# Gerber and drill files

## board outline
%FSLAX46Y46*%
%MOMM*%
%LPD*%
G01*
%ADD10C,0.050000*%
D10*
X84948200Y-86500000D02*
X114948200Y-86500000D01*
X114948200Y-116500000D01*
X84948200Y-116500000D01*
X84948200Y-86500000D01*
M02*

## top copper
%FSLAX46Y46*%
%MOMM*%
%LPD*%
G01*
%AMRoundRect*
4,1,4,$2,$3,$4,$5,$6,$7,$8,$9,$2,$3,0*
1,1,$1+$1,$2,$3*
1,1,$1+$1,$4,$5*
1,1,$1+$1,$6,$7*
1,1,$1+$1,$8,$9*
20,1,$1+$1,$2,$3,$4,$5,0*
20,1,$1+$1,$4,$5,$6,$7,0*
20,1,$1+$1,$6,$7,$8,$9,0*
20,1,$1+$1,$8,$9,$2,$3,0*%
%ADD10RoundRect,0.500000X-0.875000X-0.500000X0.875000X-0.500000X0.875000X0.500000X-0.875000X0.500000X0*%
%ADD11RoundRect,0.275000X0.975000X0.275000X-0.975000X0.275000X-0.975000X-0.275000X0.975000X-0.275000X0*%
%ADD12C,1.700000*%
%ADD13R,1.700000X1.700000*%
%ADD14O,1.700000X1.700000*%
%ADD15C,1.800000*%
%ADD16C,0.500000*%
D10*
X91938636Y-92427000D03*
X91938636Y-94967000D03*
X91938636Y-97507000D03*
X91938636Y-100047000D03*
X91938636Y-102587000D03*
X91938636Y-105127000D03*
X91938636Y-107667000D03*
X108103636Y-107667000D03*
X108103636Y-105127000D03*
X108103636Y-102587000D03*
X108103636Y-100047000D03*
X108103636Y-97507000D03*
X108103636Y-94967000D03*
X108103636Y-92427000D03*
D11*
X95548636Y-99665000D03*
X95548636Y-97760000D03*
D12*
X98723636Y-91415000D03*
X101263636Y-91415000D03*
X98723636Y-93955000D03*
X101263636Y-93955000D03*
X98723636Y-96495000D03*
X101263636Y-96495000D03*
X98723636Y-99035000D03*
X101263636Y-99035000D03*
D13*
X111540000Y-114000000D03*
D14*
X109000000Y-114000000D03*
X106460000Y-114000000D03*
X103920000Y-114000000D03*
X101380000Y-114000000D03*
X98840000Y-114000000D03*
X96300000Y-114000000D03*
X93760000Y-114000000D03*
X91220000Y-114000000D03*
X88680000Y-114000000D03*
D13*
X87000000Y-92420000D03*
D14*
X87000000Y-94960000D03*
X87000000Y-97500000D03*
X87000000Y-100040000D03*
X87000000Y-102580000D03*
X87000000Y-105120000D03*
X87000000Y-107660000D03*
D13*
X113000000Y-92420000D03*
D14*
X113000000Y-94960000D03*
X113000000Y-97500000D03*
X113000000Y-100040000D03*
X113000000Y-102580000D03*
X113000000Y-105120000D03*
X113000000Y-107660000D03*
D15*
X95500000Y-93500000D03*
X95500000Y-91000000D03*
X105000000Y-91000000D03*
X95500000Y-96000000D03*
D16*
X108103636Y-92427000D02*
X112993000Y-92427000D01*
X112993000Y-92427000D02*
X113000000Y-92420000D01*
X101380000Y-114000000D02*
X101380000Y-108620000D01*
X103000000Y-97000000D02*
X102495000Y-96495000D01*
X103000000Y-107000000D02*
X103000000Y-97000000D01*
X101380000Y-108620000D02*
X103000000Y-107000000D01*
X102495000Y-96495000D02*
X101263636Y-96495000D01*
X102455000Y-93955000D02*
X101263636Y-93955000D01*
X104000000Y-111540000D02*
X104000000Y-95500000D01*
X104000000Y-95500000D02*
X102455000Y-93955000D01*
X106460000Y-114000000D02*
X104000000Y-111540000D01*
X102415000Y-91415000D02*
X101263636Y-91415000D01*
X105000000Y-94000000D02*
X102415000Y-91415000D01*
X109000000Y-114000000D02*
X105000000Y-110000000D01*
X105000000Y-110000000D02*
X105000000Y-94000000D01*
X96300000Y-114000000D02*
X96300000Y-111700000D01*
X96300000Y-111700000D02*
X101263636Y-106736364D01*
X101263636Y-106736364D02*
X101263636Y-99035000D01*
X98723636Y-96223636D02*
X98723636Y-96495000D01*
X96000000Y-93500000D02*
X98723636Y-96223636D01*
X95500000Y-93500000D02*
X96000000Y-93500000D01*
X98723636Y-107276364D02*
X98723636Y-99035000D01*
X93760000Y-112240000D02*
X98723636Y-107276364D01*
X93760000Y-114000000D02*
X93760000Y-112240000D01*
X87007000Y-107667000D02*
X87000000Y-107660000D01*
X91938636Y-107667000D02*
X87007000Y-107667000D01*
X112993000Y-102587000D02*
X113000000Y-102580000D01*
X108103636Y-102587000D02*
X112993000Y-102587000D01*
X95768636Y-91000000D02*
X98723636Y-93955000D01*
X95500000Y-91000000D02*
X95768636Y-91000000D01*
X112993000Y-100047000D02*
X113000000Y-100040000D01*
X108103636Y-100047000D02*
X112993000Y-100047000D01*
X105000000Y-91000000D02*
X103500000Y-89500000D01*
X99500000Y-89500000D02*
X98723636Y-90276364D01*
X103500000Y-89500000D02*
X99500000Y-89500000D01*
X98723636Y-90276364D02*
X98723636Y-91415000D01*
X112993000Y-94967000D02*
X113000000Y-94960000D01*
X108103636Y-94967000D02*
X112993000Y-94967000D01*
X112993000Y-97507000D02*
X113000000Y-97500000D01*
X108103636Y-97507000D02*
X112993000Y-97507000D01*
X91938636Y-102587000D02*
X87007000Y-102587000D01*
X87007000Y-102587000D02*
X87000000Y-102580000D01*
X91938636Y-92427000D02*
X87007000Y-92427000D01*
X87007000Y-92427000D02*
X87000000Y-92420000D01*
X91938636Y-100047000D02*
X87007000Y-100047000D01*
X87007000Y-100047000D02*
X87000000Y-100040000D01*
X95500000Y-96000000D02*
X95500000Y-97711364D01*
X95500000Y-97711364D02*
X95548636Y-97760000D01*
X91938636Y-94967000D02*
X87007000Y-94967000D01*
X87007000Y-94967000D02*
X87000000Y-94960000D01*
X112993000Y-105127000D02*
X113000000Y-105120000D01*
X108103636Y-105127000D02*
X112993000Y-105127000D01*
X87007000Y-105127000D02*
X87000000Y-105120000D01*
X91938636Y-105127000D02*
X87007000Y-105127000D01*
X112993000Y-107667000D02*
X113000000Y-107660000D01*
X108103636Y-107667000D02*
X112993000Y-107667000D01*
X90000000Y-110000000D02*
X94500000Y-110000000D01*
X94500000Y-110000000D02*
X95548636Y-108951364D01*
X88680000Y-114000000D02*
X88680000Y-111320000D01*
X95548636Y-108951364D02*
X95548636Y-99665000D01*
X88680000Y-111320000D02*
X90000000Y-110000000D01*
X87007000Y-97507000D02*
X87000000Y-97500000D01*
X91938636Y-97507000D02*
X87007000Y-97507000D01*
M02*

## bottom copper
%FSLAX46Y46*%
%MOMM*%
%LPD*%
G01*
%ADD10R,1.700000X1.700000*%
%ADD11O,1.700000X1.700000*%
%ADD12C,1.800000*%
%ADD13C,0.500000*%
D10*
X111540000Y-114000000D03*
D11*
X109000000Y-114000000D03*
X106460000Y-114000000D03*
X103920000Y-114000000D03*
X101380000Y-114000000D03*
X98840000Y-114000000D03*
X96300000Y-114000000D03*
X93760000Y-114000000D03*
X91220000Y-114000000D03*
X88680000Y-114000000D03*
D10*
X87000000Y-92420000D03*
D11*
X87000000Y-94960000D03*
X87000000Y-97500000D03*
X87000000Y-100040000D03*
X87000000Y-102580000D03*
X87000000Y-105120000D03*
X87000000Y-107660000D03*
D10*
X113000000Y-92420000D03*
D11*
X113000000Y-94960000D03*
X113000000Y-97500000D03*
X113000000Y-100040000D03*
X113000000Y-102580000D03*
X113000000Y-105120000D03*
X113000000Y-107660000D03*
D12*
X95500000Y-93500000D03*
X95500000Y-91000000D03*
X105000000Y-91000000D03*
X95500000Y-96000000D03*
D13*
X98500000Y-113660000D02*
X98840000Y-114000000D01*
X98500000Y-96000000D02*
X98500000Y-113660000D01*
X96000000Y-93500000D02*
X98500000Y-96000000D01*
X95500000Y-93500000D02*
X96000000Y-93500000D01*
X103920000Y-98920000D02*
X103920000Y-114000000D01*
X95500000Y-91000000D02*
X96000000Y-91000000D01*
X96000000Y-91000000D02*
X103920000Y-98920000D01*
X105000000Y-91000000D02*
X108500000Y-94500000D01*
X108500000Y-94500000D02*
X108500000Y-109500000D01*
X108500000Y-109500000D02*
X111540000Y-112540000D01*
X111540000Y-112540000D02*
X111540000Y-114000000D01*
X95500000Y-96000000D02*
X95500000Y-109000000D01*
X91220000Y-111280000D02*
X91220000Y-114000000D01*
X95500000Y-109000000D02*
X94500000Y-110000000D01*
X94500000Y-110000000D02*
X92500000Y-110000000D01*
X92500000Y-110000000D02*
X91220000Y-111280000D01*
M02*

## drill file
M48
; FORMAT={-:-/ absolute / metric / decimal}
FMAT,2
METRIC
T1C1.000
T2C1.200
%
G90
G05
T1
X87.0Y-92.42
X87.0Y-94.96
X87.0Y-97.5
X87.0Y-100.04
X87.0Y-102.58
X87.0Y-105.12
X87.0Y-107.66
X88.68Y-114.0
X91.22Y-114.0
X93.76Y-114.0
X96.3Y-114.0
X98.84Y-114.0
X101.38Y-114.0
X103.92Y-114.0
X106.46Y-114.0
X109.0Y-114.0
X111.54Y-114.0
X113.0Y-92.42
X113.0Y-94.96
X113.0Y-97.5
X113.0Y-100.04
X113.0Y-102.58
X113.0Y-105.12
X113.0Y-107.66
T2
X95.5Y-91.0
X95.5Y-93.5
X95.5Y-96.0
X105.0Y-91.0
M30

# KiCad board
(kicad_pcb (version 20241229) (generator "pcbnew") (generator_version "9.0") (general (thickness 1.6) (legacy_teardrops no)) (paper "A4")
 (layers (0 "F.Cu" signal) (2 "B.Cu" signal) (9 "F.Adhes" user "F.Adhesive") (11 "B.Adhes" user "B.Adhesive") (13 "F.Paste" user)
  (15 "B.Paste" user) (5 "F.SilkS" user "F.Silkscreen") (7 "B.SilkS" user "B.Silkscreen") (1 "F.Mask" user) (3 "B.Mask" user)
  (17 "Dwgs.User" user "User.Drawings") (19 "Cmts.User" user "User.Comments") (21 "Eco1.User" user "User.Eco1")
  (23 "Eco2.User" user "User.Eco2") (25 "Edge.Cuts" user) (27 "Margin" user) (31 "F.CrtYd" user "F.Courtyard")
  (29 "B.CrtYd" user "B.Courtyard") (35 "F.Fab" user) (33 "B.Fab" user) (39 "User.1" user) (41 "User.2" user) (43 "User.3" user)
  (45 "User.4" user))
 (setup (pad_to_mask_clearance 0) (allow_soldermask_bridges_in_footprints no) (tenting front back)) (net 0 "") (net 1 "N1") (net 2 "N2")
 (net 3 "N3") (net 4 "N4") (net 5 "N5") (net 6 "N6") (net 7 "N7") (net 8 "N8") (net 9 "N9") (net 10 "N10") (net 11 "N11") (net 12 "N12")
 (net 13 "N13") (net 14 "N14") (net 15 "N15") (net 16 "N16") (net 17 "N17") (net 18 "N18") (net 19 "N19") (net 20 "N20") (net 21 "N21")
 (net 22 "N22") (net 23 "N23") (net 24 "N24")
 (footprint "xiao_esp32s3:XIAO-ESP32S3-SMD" (layer "F.Cu") (at 100 100)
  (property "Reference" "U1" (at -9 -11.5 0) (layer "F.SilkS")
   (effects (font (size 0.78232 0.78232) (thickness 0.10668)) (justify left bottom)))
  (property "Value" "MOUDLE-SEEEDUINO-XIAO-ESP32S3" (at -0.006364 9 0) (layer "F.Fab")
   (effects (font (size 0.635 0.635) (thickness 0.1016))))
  (pad "1" smd roundrect (at -8.061364 -7.573) (size 2.75 2) (layers "F.Cu" "F.Mask" "F.Paste") (roundrect_rratio 0.25) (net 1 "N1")
   (solder_mask_margin 0.0508) (thermal_bridge_angle 45))
  (pad "2" smd roundrect (at -8.061364 -5.033) (size 2.75 2) (layers "F.Cu" "F.Mask" "F.Paste") (roundrect_rratio 0.25) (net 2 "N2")
   (solder_mask_margin 0.0508) (thermal_bridge_angle 45))
  (pad "3" smd roundrect (at -8.061364 -2.493) (size 2.75 2) (layers "F.Cu" "F.Mask" "F.Paste") (roundrect_rratio 0.25) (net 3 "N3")
   (solder_mask_margin 0.0508) (thermal_bridge_angle 45))
  (pad "4" smd roundrect (at -8.061364 0.047) (size 2.75 2) (layers "F.Cu" "F.Mask" "F.Paste") (roundrect_rratio 0.25) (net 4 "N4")
   (solder_mask_margin 0.0508) (thermal_bridge_angle 45))
  (pad "5" smd roundrect (at -8.061364 2.587) (size 2.75 2) (layers "F.Cu" "F.Mask" "F.Paste") (roundrect_rratio 0.25) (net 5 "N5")
   (solder_mask_margin 0.0508) (thermal_bridge_angle 45))
  (pad "6" smd roundrect (at -8.061364 5.127) (size 2.75 2) (layers "F.Cu" "F.Mask" "F.Paste") (roundrect_rratio 0.25) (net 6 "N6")
   (solder_mask_margin 0.0508) (thermal_bridge_angle 45))
  (pad "7" smd roundrect (at -8.061364 7.667) (size 2.75 2) (layers "F.Cu" "F.Mask" "F.Paste") (roundrect_rratio 0.25) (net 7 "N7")
   (solder_mask_margin 0.0508) (thermal_bridge_angle 45))
  (pad "8" smd roundrect (at 8.103636 7.667) (size 2.75 2) (layers "F.Cu" "F.Mask" "F.Paste") (roundrect_rratio 0.25) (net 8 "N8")
   (solder_mask_margin 0.0508) (thermal_bridge_angle 45))
  (pad "9" smd roundrect (at 8.103636 5.127) (size 2.75 2) (layers "F.Cu" "F.Mask" "F.Paste") (roundrect_rratio 0.25) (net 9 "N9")
   (solder_mask_margin 0.0508) (thermal_bridge_angle 45))
  (pad "10" smd roundrect (at 8.103636 2.587) (size 2.75 2) (layers "F.Cu" "F.Mask" "F.Paste") (roundrect_rratio 0.25) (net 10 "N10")
   (solder_mask_margin 0.0508) (thermal_bridge_angle 45))
  (pad "11" smd roundrect (at 8.103636 0.047) (size 2.75 2) (layers "F.Cu" "F.Mask" "F.Paste") (roundrect_rratio 0.25) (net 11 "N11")
   (solder_mask_margin 0.0508) (thermal_bridge_angle 45))
  (pad "12" smd roundrect (at 8.103636 -2.493) (size 2.75 2) (layers "F.Cu" "F.Mask" "F.Paste") (roundrect_rratio 0.25) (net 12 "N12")
   (solder_mask_margin 0.0508) (thermal_bridge_angle 45))
  (pad "13" smd roundrect (at 8.103636 -5.033) (size 2.75 2) (layers "F.Cu" "F.Mask" "F.Paste") (roundrect_rratio 0.25) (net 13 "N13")
   (solder_mask_margin 0.0508) (thermal_bridge_angle 45))
  (pad "14" smd roundrect (at 8.103636 -7.573) (size 2.75 2) (layers "F.Cu" "F.Mask" "F.Paste") (roundrect_rratio 0.25) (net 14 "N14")
   (solder_mask_margin 0.0508) (thermal_bridge_angle 45))
  (pad "15" smd roundrect (at -4.451364 -0.335 180) (size 2.5 1.1) (layers "F.Cu" "F.Mask" "F.Paste") (roundrect_rratio 0.25) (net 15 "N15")
   (solder_mask_margin 0.0508) (thermal_bridge_angle 45))
  (pad "16" smd roundrect (at -4.451364 -2.24 180) (size 2.5 1.1) (layers "F.Cu" "F.Mask" "F.Paste") (roundrect_rratio 0.25) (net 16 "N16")
   (solder_mask_margin 0.0508) (thermal_bridge_angle 45))
  (pad "17" smd circle (at -1.276364 -8.585) (size 1.7 1.7) (layers "F.Cu" "F.Mask" "F.Paste") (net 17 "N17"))
  (pad "18" smd circle (at 1.263636 -8.585) (size 1.7 1.7) (layers "F.Cu" "F.Mask" "F.Paste") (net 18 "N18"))
  (pad "19" smd circle (at -1.276364 -6.045) (size 1.7 1.7) (layers "F.Cu" "F.Mask" "F.Paste") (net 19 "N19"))
  (pad "20" smd circle (at 1.263636 -6.045) (size 1.7 1.7) (layers "F.Cu" "F.Mask" "F.Paste") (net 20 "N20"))
  (pad "21" smd circle (at -1.276364 -3.505) (size 1.7 1.7) (layers "F.Cu" "F.Mask" "F.Paste") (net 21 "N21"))
  (pad "22" smd circle (at 1.263636 -3.505) (size 1.7 1.7) (layers "F.Cu" "F.Mask" "F.Paste") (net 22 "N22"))
  (pad "23" smd circle (at -1.276364 -0.965) (size 1.7 1.7) (layers "F.Cu" "F.Mask" "F.Paste") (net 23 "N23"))
  (pad "24" smd circle (at 1.263636 -0.965) (size 1.7 1.7) (layers "F.Cu" "F.Mask" "F.Paste") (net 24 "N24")))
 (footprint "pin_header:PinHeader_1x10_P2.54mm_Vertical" (layer "B.Cu") (at 111.54 114 90)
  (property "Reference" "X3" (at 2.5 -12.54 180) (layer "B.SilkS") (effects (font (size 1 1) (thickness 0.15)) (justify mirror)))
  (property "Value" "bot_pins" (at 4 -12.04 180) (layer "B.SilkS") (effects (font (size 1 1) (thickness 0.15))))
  (pad "1" thru_hole rect (at 0 0 90) (size 1.7 1.7) (drill 1) (layers "*.Cu" "*.Mask") (remove_unused_layers no) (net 17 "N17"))
  (pad "2" thru_hole oval (at 0 -2.54 90) (size 1.7 1.7) (drill 1) (layers "*.Cu" "*.Mask") (remove_unused_layers no) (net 18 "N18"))
  (pad "3" thru_hole oval (at 0 -5.08 90) (size 1.7 1.7) (drill 1) (layers "*.Cu" "*.Mask") (remove_unused_layers no) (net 20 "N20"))
  (pad "4" thru_hole oval (at 0 -7.62 90) (size 1.7 1.7) (drill 1) (layers "*.Cu" "*.Mask") (remove_unused_layers no) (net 19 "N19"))
  (pad "5" thru_hole oval (at 0 -10.16 90) (size 1.7 1.7) (drill 1) (layers "*.Cu" "*.Mask") (remove_unused_layers no) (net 22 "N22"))
  (pad "6" thru_hole oval (at 0 -12.7 90) (size 1.7 1.7) (drill 1) (layers "*.Cu" "*.Mask") (remove_unused_layers no) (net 21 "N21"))
  (pad "7" thru_hole oval (at 0 -15.24 90) (size 1.7 1.7) (drill 1) (layers "*.Cu" "*.Mask") (remove_unused_layers no) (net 24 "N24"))
  (pad "8" thru_hole oval (at 0 -17.78 90) (size 1.7 1.7) (drill 1) (layers "*.Cu" "*.Mask") (remove_unused_layers no) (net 23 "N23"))
  (pad "9" thru_hole oval (at 0 -20.32 90) (size 1.7 1.7) (drill 1) (layers "*.Cu" "*.Mask") (remove_unused_layers no) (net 16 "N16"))
  (pad "10" thru_hole oval (at 0 -22.86 90) (size 1.7 1.7) (drill 1) (layers "*.Cu" "*.Mask") (remove_unused_layers no) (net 15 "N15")))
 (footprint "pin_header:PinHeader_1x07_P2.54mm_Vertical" (layer "B.Cu") (at 87 92.42 180)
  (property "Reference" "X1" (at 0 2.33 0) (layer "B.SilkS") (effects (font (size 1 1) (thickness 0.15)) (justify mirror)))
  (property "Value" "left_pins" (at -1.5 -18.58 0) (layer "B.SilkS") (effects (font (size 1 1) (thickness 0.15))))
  (pad "1" thru_hole rect (at 0 0 180) (size 1.7 1.7) (drill 1) (layers "*.Cu" "*.Mask") (remove_unused_layers no) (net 1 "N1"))
  (pad "2" thru_hole oval (at 0 -2.54 180) (size 1.7 1.7) (drill 1) (layers "*.Cu" "*.Mask") (remove_unused_layers no) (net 2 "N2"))
  (pad "3" thru_hole oval (at 0 -5.08 180) (size 1.7 1.7) (drill 1) (layers "*.Cu" "*.Mask") (remove_unused_layers no) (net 3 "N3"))
  (pad "4" thru_hole oval (at 0 -7.62 180) (size 1.7 1.7) (drill 1) (layers "*.Cu" "*.Mask") (remove_unused_layers no) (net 4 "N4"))
  (pad "5" thru_hole oval (at 0 -10.16 180) (size 1.7 1.7) (drill 1) (layers "*.Cu" "*.Mask") (remove_unused_layers no) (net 5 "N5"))
  (pad "6" thru_hole oval (at 0 -12.7 180) (size 1.7 1.7) (drill 1) (layers "*.Cu" "*.Mask") (remove_unused_layers no) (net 6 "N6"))
  (pad "7" thru_hole oval (at 0 -15.24 180) (size 1.7 1.7) (drill 1) (layers "*.Cu" "*.Mask") (remove_unused_layers no) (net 7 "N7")))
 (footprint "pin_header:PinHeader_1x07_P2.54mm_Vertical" (layer "B.Cu") (at 113 92.42 180)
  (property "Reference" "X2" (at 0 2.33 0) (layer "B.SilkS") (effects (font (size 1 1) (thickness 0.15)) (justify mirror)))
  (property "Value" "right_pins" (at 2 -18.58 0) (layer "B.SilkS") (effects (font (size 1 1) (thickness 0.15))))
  (pad "1" thru_hole rect (at 0 0 180) (size 1.7 1.7) (drill 1) (layers "*.Cu" "*.Mask") (remove_unused_layers no) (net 14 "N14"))
  (pad "2" thru_hole oval (at 0 -2.54 180) (size 1.7 1.7) (drill 1) (layers "*.Cu" "*.Mask") (remove_unused_layers no) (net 13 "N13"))
  (pad "3" thru_hole oval (at 0 -5.08 180) (size 1.7 1.7) (drill 1) (layers "*.Cu" "*.Mask") (remove_unused_layers no) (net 12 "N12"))
  (pad "4" thru_hole oval (at 0 -7.62 180) (size 1.7 1.7) (drill 1) (layers "*.Cu" "*.Mask") (remove_unused_layers no) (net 11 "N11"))
  (pad "5" thru_hole oval (at 0 -10.16 180) (size 1.7 1.7) (drill 1) (layers "*.Cu" "*.Mask") (remove_unused_layers no) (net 10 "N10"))
  (pad "6" thru_hole oval (at 0 -12.7 180) (size 1.7 1.7) (drill 1) (layers "*.Cu" "*.Mask") (remove_unused_layers no) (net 9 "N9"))
  (pad "7" thru_hole oval (at 0 -15.24 180) (size 1.7 1.7) (drill 1) (layers "*.Cu" "*.Mask") (remove_unused_layers no) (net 8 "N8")))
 (gr_rect (start 84.9482 86.5) (end 114.9482 116.5) (stroke (width 0.05) (type default)) (fill no) (layer "Edge.Cuts"))
 (segment (start 108.103636 92.427) (end 112.993 92.427) (width 0.5) (layer "F.Cu") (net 14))
 (segment (start 112.993 92.427) (end 113 92.42) (width 0.5) (layer "F.Cu") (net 14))
 (segment (start 101.38 114) (end 101.38 108.62) (width 0.5) (layer "F.Cu") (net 22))
 (segment (start 103 97) (end 102.495 96.495) (width 0.5) (layer "F.Cu") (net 22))
 (segment (start 103 107) (end 103 97) (width 0.5) (layer "F.Cu") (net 22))
 (segment (start 101.38 108.62) (end 103 107) (width 0.5) (layer "F.Cu") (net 22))
 (segment (start 102.495 96.495) (end 101.263636 96.495) (width 0.5) (layer "F.Cu") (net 22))
 (segment (start 102.455 93.955) (end 101.263636 93.955) (width 0.5) (layer "F.Cu") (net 20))
 (segment (start 104 111.54) (end 104 95.5) (width 0.5) (layer "F.Cu") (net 20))
 (segment (start 104 95.5) (end 102.455 93.955) (width 0.5) (layer "F.Cu") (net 20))
 (segment (start 106.46 114) (end 104 111.54) (width 0.5) (layer "F.Cu") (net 20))
 (segment (start 102.415 91.415) (end 101.263636 91.415) (width 0.5) (layer "F.Cu") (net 18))
 (segment (start 105 94) (end 102.415 91.415) (width 0.5) (layer "F.Cu") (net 18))
 (segment (start 109 114) (end 105 110) (width 0.5) (layer "F.Cu") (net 18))
 (segment (start 105 110) (end 105 94) (width 0.5) (layer "F.Cu") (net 18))
 (segment (start 96.3 114) (end 96.3 111.7) (width 0.5) (layer "F.Cu") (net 24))
 (segment (start 96.3 111.7) (end 101.263636 106.736364) (width 0.5) (layer "F.Cu") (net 24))
 (segment (start 101.263636 106.736364) (end 101.263636 99.035) (width 0.5) (layer "F.Cu") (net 24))
 (segment (start 98.723636 96.223636) (end 98.723636 96.495) (width 0.5) (layer "F.Cu") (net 21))
 (segment (start 96 93.5) (end 98.723636 96.223636) (width 0.5) (layer "F.Cu") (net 21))
 (segment (start 95.5 93.5) (end 96 93.5) (width 0.5) (layer "F.Cu") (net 21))
 (via (at 95.5 93.5) (size 1.8) (drill 1.2) (layers "F.Cu" "B.Cu") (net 21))
 (segment (start 98.5 113.66) (end 98.84 114) (width 0.5) (layer "B.Cu") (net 21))
 (segment (start 98.5 96) (end 98.5 113.66) (width 0.5) (layer "B.Cu") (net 21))
 (segment (start 96 93.5) (end 98.5 96) (width 0.5) (layer "B.Cu") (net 21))
 (segment (start 95.5 93.5) (end 96 93.5) (width 0.5) (layer "B.Cu") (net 21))
 (segment (start 98.723636 107.276364) (end 98.723636 99.035) (width 0.5) (layer "F.Cu") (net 23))
 (segment (start 93.76 112.24) (end 98.723636 107.276364) (width 0.5) (layer "F.Cu") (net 23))
 (segment (start 93.76 114) (end 93.76 112.24) (width 0.5) (layer "F.Cu") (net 23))
 (segment (start 87.007 107.667) (end 87 107.66) (width 0.5) (layer "F.Cu") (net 7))
 (segment (start 91.938636 107.667) (end 87.007 107.667) (width 0.5) (layer "F.Cu") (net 7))
 (segment (start 112.993 102.587) (end 113 102.58) (width 0.5) (layer "F.Cu") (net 10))
 (segment (start 108.103636 102.587) (end 112.993 102.587) (width 0.5) (layer "F.Cu") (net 10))
 (segment (start 95.768636 91) (end 98.723636 93.955) (width 0.5) (layer "F.Cu") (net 19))
 (segment (start 95.5 91) (end 95.768636 91) (width 0.5) (layer "F.Cu") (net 19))
 (via (at 95.5 91) (size 1.8) (drill 1.2) (layers "F.Cu" "B.Cu") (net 19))
 (segment (start 103.92 98.92) (end 103.92 114) (width 0.5) (layer "B.Cu") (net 19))
 (segment (start 95.5 91) (end 96 91) (width 0.5) (layer "B.Cu") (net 19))
 (segment (start 96 91) (end 103.92 98.92) (width 0.5) (layer "B.Cu") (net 19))
 (segment (start 112.993 100.047) (end 113 100.04) (width 0.5) (layer "F.Cu") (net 11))
 (segment (start 108.103636 100.047) (end 112.993 100.047) (width 0.5) (layer "F.Cu") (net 11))
 (segment (start 105 91) (end 103.5 89.5) (width 0.5) (layer "F.Cu") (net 17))
 (segment (start 99.5 89.5) (end 98.723636 90.276364) (width 0.5) (layer "F.Cu") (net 17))
 (segment (start 103.5 89.5) (end 99.5 89.5) (width 0.5) (layer "F.Cu") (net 17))
 (segment (start 98.723636 90.276364) (end 98.723636 91.415) (width 0.5) (layer "F.Cu") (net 17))
 (via (at 105 91) (size 1.8) (drill 1.2) (layers "F.Cu" "B.Cu") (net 17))
 (segment (start 105 91) (end 108.5 94.5) (width 0.5) (layer "B.Cu") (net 17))
 (segment (start 108.5 94.5) (end 108.5 109.5) (width 0.5) (layer "B.Cu") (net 17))
 (segment (start 108.5 109.5) (end 111.54 112.54) (width 0.5) (layer "B.Cu") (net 17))
 (segment (start 111.54 112.54) (end 111.54 114) (width 0.5) (layer "B.Cu") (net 17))
 (segment (start 112.993 94.967) (end 113 94.96) (width 0.5) (layer "F.Cu") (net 13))
 (segment (start 108.103636 94.967) (end 112.993 94.967) (width 0.5) (layer "F.Cu") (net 13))
 (segment (start 112.993 97.507) (end 113 97.5) (width 0.5) (layer "F.Cu") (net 12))
 (segment (start 108.103636 97.507) (end 112.993 97.507) (width 0.5) (layer "F.Cu") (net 12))
 (segment (start 91.938636 102.587) (end 87.007 102.587) (width 0.5) (layer "F.Cu") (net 5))
 (segment (start 87.007 102.587) (end 87 102.58) (width 0.5) (layer "F.Cu") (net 5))
 (segment (start 91.938636 92.427) (end 87.007 92.427) (width 0.5) (layer "F.Cu") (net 1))
 (segment (start 87.007 92.427) (end 87 92.42) (width 0.5) (layer "F.Cu") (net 1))
 (segment (start 91.938636 100.047) (end 87.007 100.047) (width 0.5) (layer "F.Cu") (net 4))
 (segment (start 87.007 100.047) (end 87 100.04) (width 0.5) (layer "F.Cu") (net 4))
 (segment (start 95.5 96) (end 95.5 97.711364) (width 0.5) (layer "F.Cu") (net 16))
 (segment (start 95.5 97.711364) (end 95.548636 97.76) (width 0.5) (layer "F.Cu") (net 16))
 (via (at 95.5 96) (size 1.8) (drill 1.2) (layers "F.Cu" "B.Cu") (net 16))
 (segment (start 95.5 96) (end 95.5 109) (width 0.5) (layer "B.Cu") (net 16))
 (segment (start 91.22 111.28) (end 91.22 114) (width 0.5) (layer "B.Cu") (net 16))
 (segment (start 95.5 109) (end 94.5 110) (width 0.5) (layer "B.Cu") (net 16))
 (segment (start 94.5 110) (end 92.5 110) (width 0.5) (layer "B.Cu") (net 16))
 (segment (start 92.5 110) (end 91.22 111.28) (width 0.5) (layer "B.Cu") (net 16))
 (segment (start 91.938636 94.967) (end 87.007 94.967) (width 0.5) (layer "F.Cu") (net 2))
 (segment (start 87.007 94.967) (end 87 94.96) (width 0.5) (layer "F.Cu") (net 2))
 (segment (start 112.993 105.127) (end 113 105.12) (width 0.5) (layer "F.Cu") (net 9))
 (segment (start 108.103636 105.127) (end 112.993 105.127) (width 0.5) (layer "F.Cu") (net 9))
 (segment (start 87.007 105.127) (end 87 105.12) (width 0.5) (layer "F.Cu") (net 6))
 (segment (start 91.938636 105.127) (end 87.007 105.127) (width 0.5) (layer "F.Cu") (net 6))
 (segment (start 112.993 107.667) (end 113 107.66) (width 0.5) (layer "F.Cu") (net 8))
 (segment (start 108.103636 107.667) (end 112.993 107.667) (width 0.5) (layer "F.Cu") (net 8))
 (segment (start 90 110) (end 94.5 110) (width 0.5) (layer "F.Cu") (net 15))
 (segment (start 94.5 110) (end 95.548636 108.951364) (width 0.5) (layer "F.Cu") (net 15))
 (segment (start 88.68 114) (end 88.68 111.32) (width 0.5) (layer "F.Cu") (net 15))
 (segment (start 95.548636 108.951364) (end 95.548636 99.665) (width 0.5) (layer "F.Cu") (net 15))
 (segment (start 88.68 111.32) (end 90 110) (width 0.5) (layer "F.Cu") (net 15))
 (segment (start 87.007 97.507) (end 87 97.5) (width 0.5) (layer "F.Cu") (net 3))
 (segment (start 91.938636 97.507) (end 87.007 97.507) (width 0.5) (layer "F.Cu") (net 3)))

